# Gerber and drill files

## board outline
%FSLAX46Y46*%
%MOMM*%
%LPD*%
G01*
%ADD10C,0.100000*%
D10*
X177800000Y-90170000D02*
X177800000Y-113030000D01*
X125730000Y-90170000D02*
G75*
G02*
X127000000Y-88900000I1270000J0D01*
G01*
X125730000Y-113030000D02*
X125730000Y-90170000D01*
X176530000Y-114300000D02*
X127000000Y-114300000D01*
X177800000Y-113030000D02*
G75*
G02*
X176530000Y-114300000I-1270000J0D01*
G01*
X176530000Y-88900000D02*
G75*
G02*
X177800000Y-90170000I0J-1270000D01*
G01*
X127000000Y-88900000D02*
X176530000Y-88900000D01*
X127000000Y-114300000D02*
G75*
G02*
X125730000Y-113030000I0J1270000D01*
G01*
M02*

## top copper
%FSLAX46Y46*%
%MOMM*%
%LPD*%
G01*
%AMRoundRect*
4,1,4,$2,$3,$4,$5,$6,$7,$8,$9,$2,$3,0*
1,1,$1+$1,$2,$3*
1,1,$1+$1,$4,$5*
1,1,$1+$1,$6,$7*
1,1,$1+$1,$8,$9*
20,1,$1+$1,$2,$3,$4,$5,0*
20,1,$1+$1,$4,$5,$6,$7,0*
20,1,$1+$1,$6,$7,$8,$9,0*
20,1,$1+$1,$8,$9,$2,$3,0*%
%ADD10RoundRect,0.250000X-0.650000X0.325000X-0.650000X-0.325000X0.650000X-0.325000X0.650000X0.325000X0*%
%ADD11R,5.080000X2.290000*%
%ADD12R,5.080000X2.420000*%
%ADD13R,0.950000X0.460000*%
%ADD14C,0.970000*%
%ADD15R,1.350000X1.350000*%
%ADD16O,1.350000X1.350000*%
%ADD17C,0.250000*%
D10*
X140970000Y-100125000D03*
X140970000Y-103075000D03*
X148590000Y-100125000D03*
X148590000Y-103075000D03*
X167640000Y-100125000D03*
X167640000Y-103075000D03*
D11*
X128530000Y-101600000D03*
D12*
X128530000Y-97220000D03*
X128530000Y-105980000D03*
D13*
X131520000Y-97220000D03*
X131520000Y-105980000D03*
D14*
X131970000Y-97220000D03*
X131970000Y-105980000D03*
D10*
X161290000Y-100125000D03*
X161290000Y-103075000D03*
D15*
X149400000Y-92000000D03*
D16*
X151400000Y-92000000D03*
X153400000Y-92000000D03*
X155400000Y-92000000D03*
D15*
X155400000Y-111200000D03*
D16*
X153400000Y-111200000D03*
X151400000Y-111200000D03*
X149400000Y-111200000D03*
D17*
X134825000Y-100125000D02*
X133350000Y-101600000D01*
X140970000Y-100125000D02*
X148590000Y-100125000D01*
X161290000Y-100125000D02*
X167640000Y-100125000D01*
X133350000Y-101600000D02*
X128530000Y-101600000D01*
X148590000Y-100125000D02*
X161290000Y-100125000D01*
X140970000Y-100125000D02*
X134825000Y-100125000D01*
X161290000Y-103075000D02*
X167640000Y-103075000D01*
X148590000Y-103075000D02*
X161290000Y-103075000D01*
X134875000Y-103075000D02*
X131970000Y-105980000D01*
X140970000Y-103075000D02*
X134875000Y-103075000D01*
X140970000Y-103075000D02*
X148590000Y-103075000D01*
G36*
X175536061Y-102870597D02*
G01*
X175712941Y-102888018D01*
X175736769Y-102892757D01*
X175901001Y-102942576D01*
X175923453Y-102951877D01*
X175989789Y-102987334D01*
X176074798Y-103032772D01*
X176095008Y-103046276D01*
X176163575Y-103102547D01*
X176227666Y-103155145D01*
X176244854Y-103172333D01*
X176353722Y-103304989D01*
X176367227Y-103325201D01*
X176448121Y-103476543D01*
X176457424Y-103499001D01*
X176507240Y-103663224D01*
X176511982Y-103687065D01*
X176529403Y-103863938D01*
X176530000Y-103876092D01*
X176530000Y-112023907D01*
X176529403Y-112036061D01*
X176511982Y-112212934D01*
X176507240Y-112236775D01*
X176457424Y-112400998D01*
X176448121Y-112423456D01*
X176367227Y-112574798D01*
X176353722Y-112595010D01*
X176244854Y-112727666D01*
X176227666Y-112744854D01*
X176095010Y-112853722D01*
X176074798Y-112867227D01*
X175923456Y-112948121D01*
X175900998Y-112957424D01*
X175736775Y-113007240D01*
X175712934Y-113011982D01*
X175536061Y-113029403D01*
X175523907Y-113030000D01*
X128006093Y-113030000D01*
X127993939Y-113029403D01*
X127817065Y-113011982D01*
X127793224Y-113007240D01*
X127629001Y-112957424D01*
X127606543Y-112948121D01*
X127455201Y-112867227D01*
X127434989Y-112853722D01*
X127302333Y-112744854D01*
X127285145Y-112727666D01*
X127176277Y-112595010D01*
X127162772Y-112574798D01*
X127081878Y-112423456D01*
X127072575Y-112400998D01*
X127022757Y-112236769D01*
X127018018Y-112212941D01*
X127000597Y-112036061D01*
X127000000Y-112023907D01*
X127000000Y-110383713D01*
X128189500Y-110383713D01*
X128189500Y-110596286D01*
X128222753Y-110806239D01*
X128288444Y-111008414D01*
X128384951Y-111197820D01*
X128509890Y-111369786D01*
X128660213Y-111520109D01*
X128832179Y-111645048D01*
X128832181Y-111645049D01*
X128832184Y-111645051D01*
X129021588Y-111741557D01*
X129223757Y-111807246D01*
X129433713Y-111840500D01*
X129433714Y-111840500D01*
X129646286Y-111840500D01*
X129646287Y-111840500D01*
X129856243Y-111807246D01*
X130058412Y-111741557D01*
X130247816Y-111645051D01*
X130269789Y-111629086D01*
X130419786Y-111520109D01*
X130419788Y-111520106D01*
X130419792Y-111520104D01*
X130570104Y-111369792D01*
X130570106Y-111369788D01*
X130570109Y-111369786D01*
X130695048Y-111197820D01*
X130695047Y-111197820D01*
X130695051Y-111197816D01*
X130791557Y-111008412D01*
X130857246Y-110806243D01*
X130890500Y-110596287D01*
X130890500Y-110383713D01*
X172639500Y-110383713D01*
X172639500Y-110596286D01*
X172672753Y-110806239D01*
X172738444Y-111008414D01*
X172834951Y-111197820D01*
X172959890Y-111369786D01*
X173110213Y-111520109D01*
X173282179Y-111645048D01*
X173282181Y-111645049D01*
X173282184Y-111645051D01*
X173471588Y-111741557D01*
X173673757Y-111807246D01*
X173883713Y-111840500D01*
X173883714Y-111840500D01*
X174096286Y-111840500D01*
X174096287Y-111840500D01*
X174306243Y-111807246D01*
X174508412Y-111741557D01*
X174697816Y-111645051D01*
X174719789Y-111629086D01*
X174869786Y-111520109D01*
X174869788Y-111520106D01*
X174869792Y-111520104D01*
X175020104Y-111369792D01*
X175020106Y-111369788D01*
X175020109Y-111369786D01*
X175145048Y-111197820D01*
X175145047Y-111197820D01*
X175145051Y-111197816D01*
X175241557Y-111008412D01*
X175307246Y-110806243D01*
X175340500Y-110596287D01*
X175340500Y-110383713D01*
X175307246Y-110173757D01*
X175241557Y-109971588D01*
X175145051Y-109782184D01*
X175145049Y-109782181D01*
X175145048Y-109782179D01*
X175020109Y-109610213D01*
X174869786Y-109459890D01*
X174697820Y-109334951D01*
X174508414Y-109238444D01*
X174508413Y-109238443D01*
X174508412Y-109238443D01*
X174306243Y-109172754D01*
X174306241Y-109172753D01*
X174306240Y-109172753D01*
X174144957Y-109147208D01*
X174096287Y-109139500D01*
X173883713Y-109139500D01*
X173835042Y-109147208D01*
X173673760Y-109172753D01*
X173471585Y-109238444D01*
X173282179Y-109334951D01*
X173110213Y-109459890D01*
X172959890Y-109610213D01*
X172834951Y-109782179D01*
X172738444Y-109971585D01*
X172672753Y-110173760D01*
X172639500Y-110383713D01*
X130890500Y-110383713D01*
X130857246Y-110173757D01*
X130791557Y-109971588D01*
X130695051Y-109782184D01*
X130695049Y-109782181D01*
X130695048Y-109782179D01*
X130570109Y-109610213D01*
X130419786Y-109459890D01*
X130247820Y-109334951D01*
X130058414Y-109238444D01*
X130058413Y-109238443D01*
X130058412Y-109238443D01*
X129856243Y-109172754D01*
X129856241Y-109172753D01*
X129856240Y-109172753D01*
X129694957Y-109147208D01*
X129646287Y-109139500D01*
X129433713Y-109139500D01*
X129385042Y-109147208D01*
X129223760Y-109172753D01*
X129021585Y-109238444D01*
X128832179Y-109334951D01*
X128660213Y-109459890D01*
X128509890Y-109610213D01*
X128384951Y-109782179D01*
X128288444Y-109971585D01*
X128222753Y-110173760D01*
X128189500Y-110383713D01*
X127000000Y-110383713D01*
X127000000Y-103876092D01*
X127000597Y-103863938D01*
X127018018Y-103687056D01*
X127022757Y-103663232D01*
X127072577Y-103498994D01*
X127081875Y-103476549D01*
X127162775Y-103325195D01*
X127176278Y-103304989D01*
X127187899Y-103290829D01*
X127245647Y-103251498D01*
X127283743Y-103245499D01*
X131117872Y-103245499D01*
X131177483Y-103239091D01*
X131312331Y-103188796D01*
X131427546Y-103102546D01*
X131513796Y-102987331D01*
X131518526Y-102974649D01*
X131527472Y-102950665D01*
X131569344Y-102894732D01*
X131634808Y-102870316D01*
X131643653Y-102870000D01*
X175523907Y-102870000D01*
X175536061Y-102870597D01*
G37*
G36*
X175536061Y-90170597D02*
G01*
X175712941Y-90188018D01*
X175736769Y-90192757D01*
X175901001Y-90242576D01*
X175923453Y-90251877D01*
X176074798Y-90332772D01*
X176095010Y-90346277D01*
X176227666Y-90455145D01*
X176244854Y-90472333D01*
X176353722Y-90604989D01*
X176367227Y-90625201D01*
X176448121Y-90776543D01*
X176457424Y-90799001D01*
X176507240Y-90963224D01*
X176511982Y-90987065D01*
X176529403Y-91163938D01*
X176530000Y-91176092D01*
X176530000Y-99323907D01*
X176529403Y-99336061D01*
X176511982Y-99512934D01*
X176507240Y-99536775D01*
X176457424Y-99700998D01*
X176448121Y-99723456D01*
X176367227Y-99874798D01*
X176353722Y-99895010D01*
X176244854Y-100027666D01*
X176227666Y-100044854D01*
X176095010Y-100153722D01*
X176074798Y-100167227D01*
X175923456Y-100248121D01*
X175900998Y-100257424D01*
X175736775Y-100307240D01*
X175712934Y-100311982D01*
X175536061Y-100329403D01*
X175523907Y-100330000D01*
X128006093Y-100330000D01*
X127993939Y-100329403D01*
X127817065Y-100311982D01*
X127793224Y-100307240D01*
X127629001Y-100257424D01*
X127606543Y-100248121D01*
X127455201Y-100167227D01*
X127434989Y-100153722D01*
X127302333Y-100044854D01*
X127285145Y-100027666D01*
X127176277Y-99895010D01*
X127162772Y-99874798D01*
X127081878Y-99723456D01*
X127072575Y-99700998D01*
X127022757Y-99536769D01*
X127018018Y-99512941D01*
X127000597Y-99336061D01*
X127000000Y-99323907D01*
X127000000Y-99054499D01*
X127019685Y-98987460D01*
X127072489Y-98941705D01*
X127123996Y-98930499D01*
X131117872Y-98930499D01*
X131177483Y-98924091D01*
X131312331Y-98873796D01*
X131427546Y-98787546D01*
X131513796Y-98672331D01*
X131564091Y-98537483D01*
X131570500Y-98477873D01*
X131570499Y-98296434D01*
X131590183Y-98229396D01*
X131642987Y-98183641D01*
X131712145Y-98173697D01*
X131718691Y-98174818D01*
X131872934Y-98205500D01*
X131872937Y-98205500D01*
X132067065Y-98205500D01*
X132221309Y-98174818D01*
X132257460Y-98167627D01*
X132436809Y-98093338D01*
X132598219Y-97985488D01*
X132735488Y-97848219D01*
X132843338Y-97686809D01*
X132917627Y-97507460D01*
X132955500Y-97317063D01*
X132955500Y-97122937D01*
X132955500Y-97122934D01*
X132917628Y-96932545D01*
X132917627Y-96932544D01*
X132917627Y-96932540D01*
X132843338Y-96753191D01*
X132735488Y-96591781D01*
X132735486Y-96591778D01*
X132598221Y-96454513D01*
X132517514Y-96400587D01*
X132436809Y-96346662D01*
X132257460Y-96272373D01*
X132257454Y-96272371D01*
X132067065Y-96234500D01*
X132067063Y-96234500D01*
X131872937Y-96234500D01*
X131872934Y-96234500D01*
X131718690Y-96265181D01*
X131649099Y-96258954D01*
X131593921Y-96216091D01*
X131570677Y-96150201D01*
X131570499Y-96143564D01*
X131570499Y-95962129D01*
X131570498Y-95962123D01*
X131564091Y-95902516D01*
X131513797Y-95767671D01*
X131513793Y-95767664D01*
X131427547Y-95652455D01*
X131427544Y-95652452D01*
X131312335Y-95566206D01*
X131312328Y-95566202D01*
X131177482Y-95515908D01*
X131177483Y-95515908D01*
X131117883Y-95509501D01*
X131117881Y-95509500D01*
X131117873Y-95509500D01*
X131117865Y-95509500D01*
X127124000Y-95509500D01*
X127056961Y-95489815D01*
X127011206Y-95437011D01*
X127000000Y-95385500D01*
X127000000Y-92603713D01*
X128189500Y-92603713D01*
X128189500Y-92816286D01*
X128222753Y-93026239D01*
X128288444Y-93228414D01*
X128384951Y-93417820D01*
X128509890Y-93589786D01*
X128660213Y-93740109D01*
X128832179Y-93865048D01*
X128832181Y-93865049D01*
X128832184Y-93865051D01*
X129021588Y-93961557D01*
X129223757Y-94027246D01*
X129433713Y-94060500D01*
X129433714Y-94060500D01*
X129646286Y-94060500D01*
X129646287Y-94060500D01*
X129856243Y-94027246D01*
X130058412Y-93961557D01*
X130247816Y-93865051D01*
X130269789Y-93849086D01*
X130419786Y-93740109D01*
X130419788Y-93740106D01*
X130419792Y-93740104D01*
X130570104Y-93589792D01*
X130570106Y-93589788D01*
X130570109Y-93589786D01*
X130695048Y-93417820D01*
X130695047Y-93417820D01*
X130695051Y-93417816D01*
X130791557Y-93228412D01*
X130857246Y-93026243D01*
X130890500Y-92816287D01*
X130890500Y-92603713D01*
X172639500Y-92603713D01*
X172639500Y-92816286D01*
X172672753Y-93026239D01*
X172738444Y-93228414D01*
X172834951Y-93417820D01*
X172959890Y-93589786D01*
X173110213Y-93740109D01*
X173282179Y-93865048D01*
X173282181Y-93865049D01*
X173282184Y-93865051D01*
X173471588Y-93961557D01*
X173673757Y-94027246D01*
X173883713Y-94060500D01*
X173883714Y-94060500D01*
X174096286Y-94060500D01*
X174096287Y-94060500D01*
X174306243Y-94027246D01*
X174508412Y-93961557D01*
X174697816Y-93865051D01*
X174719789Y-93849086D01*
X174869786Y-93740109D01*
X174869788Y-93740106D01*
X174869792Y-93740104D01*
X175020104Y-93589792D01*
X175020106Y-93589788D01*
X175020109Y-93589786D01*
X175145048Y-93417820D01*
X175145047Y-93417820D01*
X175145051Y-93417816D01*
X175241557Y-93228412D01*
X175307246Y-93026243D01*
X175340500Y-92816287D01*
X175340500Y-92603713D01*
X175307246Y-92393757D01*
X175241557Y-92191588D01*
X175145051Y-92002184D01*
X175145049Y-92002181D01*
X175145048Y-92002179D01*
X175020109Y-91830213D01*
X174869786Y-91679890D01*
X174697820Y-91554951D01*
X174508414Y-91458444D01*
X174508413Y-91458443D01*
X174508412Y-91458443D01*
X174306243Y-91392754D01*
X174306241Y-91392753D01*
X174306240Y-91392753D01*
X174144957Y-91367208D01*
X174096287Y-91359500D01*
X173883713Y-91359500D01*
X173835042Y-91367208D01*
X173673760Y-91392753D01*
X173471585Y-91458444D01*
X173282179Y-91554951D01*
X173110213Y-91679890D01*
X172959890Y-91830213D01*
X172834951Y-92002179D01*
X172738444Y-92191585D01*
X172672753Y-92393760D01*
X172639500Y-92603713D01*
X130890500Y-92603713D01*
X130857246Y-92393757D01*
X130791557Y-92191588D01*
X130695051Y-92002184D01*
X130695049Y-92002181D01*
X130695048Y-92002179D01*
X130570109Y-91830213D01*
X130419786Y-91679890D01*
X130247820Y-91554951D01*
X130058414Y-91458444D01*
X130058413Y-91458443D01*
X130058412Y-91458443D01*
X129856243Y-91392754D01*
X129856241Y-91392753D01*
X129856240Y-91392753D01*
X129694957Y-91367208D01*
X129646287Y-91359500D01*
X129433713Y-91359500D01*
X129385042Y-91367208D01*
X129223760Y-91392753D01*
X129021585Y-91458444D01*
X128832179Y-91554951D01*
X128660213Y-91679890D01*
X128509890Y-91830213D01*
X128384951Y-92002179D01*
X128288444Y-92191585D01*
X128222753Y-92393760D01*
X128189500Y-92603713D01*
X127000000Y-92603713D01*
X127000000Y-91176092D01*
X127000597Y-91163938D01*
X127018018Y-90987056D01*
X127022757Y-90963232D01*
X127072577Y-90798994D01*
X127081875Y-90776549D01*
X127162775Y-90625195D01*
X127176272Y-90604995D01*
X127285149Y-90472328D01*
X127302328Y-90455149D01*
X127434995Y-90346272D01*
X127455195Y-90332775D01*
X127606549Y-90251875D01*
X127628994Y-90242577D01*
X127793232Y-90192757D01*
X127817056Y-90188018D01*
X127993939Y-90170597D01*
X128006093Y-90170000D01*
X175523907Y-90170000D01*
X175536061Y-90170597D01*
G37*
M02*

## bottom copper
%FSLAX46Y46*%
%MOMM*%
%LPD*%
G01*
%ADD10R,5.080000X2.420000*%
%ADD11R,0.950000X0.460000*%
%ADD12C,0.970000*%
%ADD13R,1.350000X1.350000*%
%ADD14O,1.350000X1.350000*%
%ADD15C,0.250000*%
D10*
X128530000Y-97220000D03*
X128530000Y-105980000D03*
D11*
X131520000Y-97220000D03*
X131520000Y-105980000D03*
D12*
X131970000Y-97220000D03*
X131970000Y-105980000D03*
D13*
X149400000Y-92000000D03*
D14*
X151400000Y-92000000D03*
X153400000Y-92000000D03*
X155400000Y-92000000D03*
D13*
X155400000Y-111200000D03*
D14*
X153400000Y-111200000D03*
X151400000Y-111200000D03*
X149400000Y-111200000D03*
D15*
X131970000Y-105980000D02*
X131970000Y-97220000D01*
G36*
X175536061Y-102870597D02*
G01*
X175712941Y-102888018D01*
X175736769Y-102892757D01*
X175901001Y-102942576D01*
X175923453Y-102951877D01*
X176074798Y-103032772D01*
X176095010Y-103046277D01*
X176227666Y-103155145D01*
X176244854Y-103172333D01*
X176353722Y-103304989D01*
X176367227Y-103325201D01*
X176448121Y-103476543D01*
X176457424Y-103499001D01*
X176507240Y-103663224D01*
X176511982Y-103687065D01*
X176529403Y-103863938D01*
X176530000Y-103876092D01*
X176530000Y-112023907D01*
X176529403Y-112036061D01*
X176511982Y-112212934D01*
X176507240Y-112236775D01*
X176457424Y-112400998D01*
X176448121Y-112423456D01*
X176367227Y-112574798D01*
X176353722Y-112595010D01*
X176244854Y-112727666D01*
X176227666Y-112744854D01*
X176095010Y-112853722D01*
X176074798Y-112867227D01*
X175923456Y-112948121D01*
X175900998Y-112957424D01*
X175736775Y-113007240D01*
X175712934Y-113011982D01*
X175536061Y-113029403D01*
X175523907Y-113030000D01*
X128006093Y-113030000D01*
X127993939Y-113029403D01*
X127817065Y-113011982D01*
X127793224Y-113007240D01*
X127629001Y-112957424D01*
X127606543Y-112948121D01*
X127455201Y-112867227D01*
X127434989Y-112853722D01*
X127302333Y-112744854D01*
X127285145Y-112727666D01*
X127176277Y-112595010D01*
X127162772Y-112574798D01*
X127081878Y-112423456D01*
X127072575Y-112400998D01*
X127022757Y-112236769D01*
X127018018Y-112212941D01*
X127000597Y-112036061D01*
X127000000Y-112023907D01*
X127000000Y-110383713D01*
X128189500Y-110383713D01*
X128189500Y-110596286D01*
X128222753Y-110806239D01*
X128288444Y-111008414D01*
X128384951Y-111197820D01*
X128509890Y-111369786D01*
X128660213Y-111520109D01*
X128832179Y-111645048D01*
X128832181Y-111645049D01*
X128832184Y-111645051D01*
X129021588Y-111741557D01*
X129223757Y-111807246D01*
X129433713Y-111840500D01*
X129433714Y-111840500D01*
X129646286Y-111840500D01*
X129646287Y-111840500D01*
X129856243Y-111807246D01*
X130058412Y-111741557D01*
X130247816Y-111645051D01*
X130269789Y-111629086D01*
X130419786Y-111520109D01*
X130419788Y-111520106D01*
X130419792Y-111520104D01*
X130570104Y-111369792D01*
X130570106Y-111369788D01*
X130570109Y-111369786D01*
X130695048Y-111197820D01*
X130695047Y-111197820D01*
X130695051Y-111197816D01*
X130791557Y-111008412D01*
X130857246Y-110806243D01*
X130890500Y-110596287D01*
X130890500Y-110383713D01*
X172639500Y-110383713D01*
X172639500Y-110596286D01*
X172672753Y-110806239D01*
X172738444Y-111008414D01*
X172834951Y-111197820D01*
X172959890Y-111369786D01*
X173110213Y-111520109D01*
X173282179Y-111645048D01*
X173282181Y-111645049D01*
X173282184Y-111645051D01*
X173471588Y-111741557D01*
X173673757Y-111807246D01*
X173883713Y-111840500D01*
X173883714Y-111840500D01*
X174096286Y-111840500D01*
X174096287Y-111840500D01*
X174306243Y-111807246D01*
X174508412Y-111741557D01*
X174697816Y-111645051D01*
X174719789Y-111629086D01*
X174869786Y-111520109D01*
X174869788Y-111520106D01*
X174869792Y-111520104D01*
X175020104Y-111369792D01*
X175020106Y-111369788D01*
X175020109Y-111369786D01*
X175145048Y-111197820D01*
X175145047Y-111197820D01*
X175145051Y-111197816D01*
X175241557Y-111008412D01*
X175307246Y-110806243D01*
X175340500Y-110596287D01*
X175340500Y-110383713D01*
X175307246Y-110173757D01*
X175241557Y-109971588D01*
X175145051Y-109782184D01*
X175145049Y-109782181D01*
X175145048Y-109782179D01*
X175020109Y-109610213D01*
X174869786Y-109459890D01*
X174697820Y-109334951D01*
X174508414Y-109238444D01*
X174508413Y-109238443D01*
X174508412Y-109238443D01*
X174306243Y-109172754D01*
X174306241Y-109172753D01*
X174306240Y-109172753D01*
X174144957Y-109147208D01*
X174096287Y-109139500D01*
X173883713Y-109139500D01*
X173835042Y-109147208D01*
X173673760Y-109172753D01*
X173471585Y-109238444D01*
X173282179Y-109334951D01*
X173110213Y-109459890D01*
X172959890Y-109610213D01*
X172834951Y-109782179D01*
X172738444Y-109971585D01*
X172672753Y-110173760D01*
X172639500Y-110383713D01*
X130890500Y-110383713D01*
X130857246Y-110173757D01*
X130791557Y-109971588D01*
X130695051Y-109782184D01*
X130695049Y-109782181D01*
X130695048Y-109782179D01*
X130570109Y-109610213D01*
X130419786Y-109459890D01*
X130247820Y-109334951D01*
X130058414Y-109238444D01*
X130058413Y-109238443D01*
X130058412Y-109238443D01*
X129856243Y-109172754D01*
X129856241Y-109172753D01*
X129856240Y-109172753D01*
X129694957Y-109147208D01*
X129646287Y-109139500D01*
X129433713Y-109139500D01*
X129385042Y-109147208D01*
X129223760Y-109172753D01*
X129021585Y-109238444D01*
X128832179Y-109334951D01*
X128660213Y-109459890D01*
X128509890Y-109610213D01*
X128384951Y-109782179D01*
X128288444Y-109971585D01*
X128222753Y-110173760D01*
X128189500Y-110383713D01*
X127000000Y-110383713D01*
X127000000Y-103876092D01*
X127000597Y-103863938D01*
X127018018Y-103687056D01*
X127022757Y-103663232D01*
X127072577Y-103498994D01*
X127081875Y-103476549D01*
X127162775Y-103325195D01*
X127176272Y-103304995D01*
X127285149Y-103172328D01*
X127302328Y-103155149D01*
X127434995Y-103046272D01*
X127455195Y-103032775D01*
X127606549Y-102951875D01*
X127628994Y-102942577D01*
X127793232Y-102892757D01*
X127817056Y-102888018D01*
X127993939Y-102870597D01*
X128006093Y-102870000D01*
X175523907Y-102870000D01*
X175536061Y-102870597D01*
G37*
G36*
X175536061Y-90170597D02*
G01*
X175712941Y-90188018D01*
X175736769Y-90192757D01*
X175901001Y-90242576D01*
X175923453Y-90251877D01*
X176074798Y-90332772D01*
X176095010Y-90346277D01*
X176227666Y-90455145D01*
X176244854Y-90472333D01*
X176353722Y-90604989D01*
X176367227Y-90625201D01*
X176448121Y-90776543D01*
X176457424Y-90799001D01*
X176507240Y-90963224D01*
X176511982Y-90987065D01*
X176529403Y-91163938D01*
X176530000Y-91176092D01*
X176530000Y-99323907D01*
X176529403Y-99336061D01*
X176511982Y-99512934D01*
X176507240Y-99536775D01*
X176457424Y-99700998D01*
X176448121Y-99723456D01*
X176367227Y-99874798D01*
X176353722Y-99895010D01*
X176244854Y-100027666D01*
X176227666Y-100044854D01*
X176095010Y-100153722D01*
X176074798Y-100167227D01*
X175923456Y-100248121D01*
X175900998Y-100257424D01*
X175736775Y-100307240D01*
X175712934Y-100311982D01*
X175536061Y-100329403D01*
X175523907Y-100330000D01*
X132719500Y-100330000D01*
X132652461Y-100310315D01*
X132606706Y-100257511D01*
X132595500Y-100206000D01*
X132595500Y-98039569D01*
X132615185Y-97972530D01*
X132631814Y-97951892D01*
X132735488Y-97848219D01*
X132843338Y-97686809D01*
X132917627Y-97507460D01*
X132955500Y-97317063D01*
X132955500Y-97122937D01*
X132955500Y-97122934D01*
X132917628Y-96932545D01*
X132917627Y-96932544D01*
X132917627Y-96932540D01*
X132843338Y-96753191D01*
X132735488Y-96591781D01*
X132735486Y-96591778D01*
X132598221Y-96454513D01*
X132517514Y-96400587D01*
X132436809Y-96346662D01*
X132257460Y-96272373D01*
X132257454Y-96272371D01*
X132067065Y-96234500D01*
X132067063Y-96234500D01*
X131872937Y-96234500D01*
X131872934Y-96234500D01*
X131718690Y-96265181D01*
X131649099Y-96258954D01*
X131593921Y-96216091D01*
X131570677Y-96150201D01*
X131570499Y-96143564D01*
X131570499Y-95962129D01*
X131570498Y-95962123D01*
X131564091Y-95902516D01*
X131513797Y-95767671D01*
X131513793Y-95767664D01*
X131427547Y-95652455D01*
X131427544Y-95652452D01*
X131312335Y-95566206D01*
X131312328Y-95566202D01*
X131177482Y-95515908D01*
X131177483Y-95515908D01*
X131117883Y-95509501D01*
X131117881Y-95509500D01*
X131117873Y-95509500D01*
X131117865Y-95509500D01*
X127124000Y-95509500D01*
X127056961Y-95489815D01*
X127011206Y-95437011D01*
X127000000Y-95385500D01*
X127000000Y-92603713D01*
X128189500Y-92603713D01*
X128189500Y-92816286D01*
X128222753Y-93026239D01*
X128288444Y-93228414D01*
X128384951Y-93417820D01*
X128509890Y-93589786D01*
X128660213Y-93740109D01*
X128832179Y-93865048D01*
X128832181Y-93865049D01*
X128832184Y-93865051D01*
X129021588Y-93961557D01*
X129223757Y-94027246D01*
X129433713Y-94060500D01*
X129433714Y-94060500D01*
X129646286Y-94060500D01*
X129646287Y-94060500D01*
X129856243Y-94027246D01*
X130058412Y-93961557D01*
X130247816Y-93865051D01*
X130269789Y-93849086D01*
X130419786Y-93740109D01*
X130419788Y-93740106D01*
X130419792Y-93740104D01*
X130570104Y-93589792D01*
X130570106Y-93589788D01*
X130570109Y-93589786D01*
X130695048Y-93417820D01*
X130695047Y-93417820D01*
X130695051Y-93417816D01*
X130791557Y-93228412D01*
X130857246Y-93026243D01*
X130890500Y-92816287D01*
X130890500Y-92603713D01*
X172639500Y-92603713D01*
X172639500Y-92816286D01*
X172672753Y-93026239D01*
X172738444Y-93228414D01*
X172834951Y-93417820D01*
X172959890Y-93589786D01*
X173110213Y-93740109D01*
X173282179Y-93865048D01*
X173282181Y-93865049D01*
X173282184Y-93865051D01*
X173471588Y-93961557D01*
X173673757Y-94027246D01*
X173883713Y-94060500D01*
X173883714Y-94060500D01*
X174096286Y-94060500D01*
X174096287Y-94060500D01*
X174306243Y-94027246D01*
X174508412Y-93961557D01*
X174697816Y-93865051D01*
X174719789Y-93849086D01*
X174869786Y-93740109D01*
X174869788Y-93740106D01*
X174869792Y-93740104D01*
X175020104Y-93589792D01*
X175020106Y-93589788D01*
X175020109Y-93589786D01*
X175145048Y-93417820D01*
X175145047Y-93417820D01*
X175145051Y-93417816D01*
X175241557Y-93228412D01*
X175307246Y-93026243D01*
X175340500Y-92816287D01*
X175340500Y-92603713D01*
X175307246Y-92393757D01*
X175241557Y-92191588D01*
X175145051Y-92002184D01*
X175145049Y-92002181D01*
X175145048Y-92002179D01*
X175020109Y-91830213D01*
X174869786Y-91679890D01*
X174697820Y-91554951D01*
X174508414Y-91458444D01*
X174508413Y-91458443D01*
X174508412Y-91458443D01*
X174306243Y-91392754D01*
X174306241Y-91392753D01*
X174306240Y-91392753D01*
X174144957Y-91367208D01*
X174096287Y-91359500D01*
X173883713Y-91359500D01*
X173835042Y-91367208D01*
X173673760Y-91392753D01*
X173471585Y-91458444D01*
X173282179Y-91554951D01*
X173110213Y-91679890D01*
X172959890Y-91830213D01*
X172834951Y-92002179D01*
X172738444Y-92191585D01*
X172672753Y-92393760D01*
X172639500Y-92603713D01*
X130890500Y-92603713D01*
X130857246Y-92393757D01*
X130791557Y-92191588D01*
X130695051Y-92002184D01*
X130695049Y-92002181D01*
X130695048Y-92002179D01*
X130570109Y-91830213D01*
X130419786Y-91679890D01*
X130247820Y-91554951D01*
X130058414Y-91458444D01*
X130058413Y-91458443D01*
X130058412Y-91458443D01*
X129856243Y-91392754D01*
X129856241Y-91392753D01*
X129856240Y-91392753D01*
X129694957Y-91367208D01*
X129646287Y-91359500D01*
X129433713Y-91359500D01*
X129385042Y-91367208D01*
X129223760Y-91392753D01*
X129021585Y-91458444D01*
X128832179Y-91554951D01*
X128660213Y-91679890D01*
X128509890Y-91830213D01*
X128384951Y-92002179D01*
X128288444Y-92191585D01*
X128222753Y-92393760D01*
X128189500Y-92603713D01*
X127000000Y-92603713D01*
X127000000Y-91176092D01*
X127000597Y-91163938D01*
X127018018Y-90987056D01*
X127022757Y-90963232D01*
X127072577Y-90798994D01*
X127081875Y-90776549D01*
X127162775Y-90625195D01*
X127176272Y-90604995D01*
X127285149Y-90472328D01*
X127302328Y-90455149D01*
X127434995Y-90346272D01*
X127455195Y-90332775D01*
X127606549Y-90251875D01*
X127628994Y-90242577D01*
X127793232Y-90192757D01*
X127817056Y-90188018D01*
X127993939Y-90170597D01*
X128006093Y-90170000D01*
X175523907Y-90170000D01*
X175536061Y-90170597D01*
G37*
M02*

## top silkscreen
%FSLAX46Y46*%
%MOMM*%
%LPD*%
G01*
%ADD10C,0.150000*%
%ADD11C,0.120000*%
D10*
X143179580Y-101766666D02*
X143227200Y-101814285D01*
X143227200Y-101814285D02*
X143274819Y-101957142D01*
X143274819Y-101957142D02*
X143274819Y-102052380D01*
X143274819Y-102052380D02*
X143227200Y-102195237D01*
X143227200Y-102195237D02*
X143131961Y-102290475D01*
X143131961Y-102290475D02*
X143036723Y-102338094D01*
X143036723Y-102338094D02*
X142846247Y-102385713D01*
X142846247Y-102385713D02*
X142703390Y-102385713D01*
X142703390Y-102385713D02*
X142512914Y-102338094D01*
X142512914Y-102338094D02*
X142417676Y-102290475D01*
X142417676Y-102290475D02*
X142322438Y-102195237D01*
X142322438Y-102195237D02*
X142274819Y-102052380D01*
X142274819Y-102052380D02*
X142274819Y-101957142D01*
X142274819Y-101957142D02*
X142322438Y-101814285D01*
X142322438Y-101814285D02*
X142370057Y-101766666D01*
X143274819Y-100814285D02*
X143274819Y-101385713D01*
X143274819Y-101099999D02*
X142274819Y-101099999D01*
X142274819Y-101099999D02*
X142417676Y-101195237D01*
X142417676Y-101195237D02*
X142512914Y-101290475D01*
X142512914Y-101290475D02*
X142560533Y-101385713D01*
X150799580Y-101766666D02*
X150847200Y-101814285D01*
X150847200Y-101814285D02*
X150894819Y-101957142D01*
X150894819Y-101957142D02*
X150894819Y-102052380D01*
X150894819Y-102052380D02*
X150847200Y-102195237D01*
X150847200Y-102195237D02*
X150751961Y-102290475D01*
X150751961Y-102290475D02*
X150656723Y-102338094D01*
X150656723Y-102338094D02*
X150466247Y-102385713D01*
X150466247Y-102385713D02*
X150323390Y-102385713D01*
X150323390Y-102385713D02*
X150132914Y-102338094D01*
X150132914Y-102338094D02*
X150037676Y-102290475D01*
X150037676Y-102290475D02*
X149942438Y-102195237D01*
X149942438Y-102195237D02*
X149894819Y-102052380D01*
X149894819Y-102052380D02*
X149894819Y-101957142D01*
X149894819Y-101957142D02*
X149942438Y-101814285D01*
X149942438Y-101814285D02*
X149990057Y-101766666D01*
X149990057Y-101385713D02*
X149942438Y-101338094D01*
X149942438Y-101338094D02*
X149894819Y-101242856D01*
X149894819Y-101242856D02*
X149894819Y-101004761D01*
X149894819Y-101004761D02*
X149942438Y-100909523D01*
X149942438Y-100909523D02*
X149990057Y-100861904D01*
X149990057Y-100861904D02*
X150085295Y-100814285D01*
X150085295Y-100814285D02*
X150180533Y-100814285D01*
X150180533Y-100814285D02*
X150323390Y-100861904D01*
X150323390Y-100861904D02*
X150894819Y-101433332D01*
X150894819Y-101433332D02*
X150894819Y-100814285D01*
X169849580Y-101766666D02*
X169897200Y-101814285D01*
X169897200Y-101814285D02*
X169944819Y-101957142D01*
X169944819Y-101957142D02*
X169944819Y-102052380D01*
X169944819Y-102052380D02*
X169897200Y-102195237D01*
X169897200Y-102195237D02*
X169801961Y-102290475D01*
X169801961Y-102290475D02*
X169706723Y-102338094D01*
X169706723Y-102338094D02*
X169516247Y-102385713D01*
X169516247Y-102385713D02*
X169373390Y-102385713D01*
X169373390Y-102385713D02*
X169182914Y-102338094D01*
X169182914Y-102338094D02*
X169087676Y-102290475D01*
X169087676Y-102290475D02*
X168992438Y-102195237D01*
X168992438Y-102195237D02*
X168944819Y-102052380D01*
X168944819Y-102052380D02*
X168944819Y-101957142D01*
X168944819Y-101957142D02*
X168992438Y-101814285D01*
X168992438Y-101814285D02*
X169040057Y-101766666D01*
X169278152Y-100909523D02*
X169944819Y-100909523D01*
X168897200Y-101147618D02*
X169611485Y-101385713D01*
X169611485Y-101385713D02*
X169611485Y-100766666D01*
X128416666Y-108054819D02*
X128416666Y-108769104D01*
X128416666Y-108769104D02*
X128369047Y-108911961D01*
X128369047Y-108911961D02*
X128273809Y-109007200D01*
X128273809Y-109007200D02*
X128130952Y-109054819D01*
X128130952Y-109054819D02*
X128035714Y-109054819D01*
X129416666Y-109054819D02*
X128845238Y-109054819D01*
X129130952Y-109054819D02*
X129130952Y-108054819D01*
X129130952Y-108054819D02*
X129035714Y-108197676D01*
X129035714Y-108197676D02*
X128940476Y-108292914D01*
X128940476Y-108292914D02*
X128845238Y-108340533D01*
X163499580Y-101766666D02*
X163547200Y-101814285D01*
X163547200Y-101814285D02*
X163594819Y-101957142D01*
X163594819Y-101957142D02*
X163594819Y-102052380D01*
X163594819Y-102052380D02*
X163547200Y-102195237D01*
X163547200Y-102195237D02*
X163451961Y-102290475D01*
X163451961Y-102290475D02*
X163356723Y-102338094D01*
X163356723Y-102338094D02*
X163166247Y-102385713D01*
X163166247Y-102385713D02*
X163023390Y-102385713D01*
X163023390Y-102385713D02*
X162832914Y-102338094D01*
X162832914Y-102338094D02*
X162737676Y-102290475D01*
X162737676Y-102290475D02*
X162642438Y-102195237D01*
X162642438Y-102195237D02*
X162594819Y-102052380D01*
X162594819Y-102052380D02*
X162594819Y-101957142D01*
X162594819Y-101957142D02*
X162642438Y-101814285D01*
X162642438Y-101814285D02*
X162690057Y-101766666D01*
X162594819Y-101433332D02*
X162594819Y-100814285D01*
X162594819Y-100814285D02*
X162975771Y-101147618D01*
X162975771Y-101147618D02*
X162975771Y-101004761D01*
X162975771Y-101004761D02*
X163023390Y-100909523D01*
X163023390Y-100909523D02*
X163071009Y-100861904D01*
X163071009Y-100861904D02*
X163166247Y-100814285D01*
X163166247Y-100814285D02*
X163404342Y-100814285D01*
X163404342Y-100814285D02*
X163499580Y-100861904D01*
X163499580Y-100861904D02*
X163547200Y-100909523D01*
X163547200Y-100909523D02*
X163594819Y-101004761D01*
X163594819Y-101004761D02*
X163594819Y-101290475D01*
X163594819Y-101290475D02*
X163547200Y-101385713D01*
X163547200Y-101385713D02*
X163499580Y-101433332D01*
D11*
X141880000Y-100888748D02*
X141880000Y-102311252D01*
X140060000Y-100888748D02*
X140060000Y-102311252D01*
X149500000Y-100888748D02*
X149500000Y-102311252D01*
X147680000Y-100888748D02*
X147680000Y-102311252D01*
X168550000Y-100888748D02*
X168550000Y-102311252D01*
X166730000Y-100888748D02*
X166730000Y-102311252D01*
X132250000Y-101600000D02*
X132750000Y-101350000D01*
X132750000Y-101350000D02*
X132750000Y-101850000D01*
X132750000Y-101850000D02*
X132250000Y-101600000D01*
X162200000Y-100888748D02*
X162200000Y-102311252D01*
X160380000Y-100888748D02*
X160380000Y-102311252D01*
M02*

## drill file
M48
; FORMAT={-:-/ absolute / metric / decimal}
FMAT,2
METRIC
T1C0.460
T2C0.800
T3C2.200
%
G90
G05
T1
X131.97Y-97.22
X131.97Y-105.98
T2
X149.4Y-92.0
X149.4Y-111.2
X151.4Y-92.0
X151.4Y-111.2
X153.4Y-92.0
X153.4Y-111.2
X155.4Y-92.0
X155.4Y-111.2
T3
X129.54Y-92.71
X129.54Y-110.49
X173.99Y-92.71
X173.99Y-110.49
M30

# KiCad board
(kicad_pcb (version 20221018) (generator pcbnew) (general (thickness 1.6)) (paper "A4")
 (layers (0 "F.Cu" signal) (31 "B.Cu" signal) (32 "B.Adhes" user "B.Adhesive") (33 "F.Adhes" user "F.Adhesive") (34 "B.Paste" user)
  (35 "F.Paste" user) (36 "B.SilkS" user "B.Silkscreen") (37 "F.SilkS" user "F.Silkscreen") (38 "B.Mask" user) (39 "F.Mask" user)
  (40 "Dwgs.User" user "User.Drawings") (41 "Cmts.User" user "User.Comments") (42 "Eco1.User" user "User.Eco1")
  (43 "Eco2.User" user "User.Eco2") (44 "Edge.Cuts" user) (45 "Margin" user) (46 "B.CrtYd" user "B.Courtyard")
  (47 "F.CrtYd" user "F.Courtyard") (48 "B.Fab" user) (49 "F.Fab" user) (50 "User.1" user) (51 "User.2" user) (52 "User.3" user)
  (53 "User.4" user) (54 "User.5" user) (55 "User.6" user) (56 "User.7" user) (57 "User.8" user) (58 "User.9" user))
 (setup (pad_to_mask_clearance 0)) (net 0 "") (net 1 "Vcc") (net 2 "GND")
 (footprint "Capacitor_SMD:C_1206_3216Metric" (layer "F.Cu") (at 140.97 101.6 -90)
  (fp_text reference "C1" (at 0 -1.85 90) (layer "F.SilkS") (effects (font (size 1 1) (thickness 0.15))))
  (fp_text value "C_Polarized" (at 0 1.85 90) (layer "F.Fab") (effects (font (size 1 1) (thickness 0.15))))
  (fp_line (start -0.711252 -0.91) (end 0.711252 -0.91) (stroke (width 0.12) (type solid)) (layer "F.SilkS"))
  (fp_line (start -0.711252 0.91) (end 0.711252 0.91) (stroke (width 0.12) (type solid)) (layer "F.SilkS"))
  (pad "1" smd roundrect (at -1.475 0 270) (size 1.15 1.8) (layers "F.Cu" "F.Paste" "F.Mask") (roundrect_rratio 0.217391) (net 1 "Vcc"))
  (pad "2" smd roundrect (at 1.475 0 270) (size 1.15 1.8) (layers "F.Cu" "F.Paste" "F.Mask") (roundrect_rratio 0.217391) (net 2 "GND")))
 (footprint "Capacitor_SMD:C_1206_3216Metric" (layer "F.Cu") (at 148.59 101.6 -90)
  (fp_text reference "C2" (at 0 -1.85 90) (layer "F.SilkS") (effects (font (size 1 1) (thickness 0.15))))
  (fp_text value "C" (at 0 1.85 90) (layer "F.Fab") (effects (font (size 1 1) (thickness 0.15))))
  (fp_line (start -0.711252 -0.91) (end 0.711252 -0.91) (stroke (width 0.12) (type solid)) (layer "F.SilkS"))
  (fp_line (start -0.711252 0.91) (end 0.711252 0.91) (stroke (width 0.12) (type solid)) (layer "F.SilkS"))
  (pad "1" smd roundrect (at -1.475 0 270) (size 1.15 1.8) (layers "F.Cu" "F.Paste" "F.Mask") (roundrect_rratio 0.217391) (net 1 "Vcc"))
  (pad "2" smd roundrect (at 1.475 0 270) (size 1.15 1.8) (layers "F.Cu" "F.Paste" "F.Mask") (roundrect_rratio 0.217391) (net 2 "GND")))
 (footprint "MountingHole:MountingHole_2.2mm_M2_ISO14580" (layer "F.Cu") (at 129.54 92.71)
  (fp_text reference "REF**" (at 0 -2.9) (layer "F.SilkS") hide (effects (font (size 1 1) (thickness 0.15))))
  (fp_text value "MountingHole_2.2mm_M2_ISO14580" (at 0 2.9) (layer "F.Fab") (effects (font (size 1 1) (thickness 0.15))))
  (pad "" np_thru_hole circle (at 0 0) (size 2.2 2.2) (drill 2.2) (layers "*.Cu" "*.Mask")))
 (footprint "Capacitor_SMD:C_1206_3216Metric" (layer "F.Cu") (at 167.64 101.6 -90)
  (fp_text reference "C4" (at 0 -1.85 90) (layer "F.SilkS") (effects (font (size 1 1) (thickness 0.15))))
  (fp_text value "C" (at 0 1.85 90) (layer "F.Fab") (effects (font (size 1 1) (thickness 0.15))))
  (fp_line (start -0.711252 -0.91) (end 0.711252 -0.91) (stroke (width 0.12) (type solid)) (layer "F.SilkS"))
  (fp_line (start -0.711252 0.91) (end 0.711252 0.91) (stroke (width 0.12) (type solid)) (layer "F.SilkS"))
  (pad "1" smd roundrect (at -1.475 0 270) (size 1.15 1.8) (layers "F.Cu" "F.Paste" "F.Mask") (roundrect_rratio 0.217391) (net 1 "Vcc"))
  (pad "2" smd roundrect (at 1.475 0 270) (size 1.15 1.8) (layers "F.Cu" "F.Paste" "F.Mask") (roundrect_rratio 0.217391) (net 2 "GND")))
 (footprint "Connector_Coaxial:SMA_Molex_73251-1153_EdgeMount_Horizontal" (layer "F.Cu") (at 130.25 101.6)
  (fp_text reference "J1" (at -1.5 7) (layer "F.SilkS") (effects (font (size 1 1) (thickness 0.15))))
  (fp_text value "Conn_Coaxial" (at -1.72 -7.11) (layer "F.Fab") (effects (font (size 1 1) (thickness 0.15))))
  (fp_line (start 2 0) (end 2.5 -0.25) (stroke (width 0.12) (type solid)) (layer "F.SilkS"))
  (fp_line (start 2.5 -0.25) (end 2.5 0.25) (stroke (width 0.12) (type solid)) (layer "F.SilkS"))
  (fp_line (start 2.5 0.25) (end 2 0) (stroke (width 0.12) (type solid)) (layer "F.SilkS"))
  (pad "1" smd rect (at -1.72 0) (size 5.08 2.29) (layers "F.Cu" "F.Paste" "F.Mask") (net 1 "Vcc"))
  (pad "2" smd rect (at -1.72 -4.38) (size 5.08 2.42) (layers "F.Cu" "F.Paste" "F.Mask") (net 2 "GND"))
  (pad "2" smd rect (at -1.72 -4.38) (size 5.08 2.42) (layers "B.Cu" "B.Paste" "B.Mask") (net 2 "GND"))
  (pad "2" smd rect (at -1.72 4.38) (size 5.08 2.42) (layers "F.Cu" "F.Paste" "F.Mask") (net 2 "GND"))
  (pad "2" smd rect (at -1.72 4.38) (size 5.08 2.42) (layers "B.Cu" "B.Paste" "B.Mask") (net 2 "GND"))
  (pad "2" smd rect (at 1.27 -4.38) (size 0.95 0.46) (layers "F.Cu") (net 2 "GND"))
  (pad "2" smd rect (at 1.27 -4.38) (size 0.95 0.46) (layers "B.Cu") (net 2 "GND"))
  (pad "2" smd rect (at 1.27 4.38) (size 0.95 0.46) (layers "F.Cu") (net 2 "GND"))
  (pad "2" smd rect (at 1.27 4.38) (size 0.95 0.46) (layers "B.Cu") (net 2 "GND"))
  (pad "2" thru_hole circle (at 1.72 -4.38) (size 0.97 0.97) (drill 0.46) (layers "*.Cu") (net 2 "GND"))
  (pad "2" thru_hole circle (at 1.72 4.38) (size 0.97 0.97) (drill 0.46) (layers "*.Cu") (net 2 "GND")))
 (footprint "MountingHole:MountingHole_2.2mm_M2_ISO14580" (layer "F.Cu") (at 173.99 92.71)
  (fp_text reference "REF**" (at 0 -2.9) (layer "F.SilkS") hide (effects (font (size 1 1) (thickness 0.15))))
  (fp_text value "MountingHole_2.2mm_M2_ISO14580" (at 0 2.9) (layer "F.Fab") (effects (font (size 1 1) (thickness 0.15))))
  (pad "" np_thru_hole circle (at 0 0) (size 2.2 2.2) (drill 2.2) (layers "*.Cu" "*.Mask")))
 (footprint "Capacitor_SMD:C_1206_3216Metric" (layer "F.Cu") (at 161.29 101.6 -90)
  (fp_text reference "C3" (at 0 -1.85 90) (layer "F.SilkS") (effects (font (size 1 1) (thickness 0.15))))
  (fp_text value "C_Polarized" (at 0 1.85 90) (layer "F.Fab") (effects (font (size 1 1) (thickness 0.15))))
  (fp_line (start -0.711252 -0.91) (end 0.711252 -0.91) (stroke (width 0.12) (type solid)) (layer "F.SilkS"))
  (fp_line (start -0.711252 0.91) (end 0.711252 0.91) (stroke (width 0.12) (type solid)) (layer "F.SilkS"))
  (pad "1" smd roundrect (at -1.475 0 270) (size 1.15 1.8) (layers "F.Cu" "F.Paste" "F.Mask") (roundrect_rratio 0.217391) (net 1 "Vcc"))
  (pad "2" smd roundrect (at 1.475 0 270) (size 1.15 1.8) (layers "F.Cu" "F.Paste" "F.Mask") (roundrect_rratio 0.217391) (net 2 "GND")))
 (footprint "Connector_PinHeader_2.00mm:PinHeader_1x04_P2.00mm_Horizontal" (layer "F.Cu") (at 149.4 92 90) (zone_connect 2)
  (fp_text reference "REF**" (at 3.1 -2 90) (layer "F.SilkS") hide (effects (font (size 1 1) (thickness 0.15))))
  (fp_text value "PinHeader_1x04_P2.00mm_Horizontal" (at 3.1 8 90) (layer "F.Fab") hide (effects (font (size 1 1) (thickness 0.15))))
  (pad "1" thru_hole rect (at 0 0 90) (size 1.35 1.35) (drill 0.8) (layers "*.Cu" "*.Mask") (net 1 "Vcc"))
  (pad "2" thru_hole oval (at 0 2 90) (size 1.35 1.35) (drill 0.8) (layers "*.Cu" "*.Mask") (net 1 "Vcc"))
  (pad "3" thru_hole oval (at 0 4 90) (size 1.35 1.35) (drill 0.8) (layers "*.Cu" "*.Mask") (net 1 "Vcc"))
  (pad "4" thru_hole oval (at 0 6 90) (size 1.35 1.35) (drill 0.8) (layers "*.Cu" "*.Mask") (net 1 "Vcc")))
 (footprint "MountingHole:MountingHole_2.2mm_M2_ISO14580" (layer "F.Cu") (at 129.54 110.49)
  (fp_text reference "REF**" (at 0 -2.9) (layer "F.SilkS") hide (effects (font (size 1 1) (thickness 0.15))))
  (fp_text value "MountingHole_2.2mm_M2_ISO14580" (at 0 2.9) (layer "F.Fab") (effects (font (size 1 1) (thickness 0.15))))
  (pad "" np_thru_hole circle (at 0 0) (size 2.2 2.2) (drill 2.2) (layers "*.Cu" "*.Mask")))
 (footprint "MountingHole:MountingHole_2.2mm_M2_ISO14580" (layer "F.Cu") (at 173.99 110.49)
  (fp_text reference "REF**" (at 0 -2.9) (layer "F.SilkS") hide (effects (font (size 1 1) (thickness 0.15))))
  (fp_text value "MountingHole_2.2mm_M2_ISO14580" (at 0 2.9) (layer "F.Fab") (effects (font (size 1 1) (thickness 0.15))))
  (pad "" np_thru_hole circle (at 0 0) (size 2.2 2.2) (drill 2.2) (layers "*.Cu" "*.Mask")))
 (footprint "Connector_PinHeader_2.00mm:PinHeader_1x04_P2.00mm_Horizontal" (layer "F.Cu") (at 155.4 111.2 -90) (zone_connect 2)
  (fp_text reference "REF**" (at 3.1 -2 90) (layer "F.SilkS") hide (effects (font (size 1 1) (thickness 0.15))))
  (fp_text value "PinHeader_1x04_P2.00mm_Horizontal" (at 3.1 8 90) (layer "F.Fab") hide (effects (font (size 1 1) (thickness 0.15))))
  (pad "1" thru_hole rect (at 0 0 270) (size 1.35 1.35) (drill 0.8) (layers "*.Cu" "*.Mask") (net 2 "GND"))
  (pad "2" thru_hole oval (at 0 2 270) (size 1.35 1.35) (drill 0.8) (layers "*.Cu" "*.Mask") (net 2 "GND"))
  (pad "3" thru_hole oval (at 0 4 270) (size 1.35 1.35) (drill 0.8) (layers "*.Cu" "*.Mask") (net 2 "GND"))
  (pad "4" thru_hole oval (at 0 6 270) (size 1.35 1.35) (drill 0.8) (layers "*.Cu" "*.Mask") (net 2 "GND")))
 (gr_line (start 177.8 90.17) (end 177.8 113.03) (stroke (width 0.1) (type default)) (layer "Edge.Cuts"))
 (gr_arc (start 125.73 90.17) (mid 126.101974 89.271974) (end 127 88.9) (stroke (width 0.1) (type default)) (layer "Edge.Cuts"))
 (gr_line (start 125.73 113.03) (end 125.73 90.17) (stroke (width 0.1) (type default)) (layer "Edge.Cuts"))
 (gr_line (start 176.53 114.3) (end 127 114.3) (stroke (width 0.1) (type default)) (layer "Edge.Cuts"))
 (gr_arc (start 177.8 113.03) (mid 177.428026 113.928026) (end 176.53 114.3) (stroke (width 0.1) (type default)) (layer "Edge.Cuts"))
 (gr_arc (start 176.53 88.9) (mid 177.428026 89.271974) (end 177.8 90.17) (stroke (width 0.1) (type default)) (layer "Edge.Cuts"))
 (gr_line (start 127 88.9) (end 176.53 88.9) (stroke (width 0.1) (type default)) (layer "Edge.Cuts"))
 (gr_arc (start 127 114.3) (mid 126.101974 113.928026) (end 125.73 113.03) (stroke (width 0.1) (type default)) (layer "Edge.Cuts"))
 (segment (start 134.825 100.125) (end 133.35 101.6) (width 0.25) (layer "F.Cu") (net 1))
 (segment (start 140.97 100.125) (end 148.59 100.125) (width 0.25) (layer "F.Cu") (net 1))
 (segment (start 161.29 100.125) (end 167.64 100.125) (width 0.25) (layer "F.Cu") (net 1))
 (segment (start 133.35 101.6) (end 128.53 101.6) (width 0.25) (layer "F.Cu") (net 1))
 (segment (start 148.59 100.125) (end 161.29 100.125) (width 0.25) (layer "F.Cu") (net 1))
 (segment (start 140.97 100.125) (end 134.825 100.125) (width 0.25) (layer "F.Cu") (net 1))
 (segment (start 161.29 103.075) (end 167.64 103.075) (width 0.25) (layer "F.Cu") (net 2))
 (segment (start 148.59 103.075) (end 161.29 103.075) (width 0.25) (layer "F.Cu") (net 2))
 (segment (start 134.875 103.075) (end 131.97 105.98) (width 0.25) (layer "F.Cu") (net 2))
 (segment (start 140.97 103.075) (end 134.875 103.075) (width 0.25) (layer "F.Cu") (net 2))
 (segment (start 140.97 103.075) (end 148.59 103.075) (width 0.25) (layer "F.Cu") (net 2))
 (segment (start 131.97 105.98) (end 131.97 97.22) (width 0.25) (layer "B.Cu") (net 2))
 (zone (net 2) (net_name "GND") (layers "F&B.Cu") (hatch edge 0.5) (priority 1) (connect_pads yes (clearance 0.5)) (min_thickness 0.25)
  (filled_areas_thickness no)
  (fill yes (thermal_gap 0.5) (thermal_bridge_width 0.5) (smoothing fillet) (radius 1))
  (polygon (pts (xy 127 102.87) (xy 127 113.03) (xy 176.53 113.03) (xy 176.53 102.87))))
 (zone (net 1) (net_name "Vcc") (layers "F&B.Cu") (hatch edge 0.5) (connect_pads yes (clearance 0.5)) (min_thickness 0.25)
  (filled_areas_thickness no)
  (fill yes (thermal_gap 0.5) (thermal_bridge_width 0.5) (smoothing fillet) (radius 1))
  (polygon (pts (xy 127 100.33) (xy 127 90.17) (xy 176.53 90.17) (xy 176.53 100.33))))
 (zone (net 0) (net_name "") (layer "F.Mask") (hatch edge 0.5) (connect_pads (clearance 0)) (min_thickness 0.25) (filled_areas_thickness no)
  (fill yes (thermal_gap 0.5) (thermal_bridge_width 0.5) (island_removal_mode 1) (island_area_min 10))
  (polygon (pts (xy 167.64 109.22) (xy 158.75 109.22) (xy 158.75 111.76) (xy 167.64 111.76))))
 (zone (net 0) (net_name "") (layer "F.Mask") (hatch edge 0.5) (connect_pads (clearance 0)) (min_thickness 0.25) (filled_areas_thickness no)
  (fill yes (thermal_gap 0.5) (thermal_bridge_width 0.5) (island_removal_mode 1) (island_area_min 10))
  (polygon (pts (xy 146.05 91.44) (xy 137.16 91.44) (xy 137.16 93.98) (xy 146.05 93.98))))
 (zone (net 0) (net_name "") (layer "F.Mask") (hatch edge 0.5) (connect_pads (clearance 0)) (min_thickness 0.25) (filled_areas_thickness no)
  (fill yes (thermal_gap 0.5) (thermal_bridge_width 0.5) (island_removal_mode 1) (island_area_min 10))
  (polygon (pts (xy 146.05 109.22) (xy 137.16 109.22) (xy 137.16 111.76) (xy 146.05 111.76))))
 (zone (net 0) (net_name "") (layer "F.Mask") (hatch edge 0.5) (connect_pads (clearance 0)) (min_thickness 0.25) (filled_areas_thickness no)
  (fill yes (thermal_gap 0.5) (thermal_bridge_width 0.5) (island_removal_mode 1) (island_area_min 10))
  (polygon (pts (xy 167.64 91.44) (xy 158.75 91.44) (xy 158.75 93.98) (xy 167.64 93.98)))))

